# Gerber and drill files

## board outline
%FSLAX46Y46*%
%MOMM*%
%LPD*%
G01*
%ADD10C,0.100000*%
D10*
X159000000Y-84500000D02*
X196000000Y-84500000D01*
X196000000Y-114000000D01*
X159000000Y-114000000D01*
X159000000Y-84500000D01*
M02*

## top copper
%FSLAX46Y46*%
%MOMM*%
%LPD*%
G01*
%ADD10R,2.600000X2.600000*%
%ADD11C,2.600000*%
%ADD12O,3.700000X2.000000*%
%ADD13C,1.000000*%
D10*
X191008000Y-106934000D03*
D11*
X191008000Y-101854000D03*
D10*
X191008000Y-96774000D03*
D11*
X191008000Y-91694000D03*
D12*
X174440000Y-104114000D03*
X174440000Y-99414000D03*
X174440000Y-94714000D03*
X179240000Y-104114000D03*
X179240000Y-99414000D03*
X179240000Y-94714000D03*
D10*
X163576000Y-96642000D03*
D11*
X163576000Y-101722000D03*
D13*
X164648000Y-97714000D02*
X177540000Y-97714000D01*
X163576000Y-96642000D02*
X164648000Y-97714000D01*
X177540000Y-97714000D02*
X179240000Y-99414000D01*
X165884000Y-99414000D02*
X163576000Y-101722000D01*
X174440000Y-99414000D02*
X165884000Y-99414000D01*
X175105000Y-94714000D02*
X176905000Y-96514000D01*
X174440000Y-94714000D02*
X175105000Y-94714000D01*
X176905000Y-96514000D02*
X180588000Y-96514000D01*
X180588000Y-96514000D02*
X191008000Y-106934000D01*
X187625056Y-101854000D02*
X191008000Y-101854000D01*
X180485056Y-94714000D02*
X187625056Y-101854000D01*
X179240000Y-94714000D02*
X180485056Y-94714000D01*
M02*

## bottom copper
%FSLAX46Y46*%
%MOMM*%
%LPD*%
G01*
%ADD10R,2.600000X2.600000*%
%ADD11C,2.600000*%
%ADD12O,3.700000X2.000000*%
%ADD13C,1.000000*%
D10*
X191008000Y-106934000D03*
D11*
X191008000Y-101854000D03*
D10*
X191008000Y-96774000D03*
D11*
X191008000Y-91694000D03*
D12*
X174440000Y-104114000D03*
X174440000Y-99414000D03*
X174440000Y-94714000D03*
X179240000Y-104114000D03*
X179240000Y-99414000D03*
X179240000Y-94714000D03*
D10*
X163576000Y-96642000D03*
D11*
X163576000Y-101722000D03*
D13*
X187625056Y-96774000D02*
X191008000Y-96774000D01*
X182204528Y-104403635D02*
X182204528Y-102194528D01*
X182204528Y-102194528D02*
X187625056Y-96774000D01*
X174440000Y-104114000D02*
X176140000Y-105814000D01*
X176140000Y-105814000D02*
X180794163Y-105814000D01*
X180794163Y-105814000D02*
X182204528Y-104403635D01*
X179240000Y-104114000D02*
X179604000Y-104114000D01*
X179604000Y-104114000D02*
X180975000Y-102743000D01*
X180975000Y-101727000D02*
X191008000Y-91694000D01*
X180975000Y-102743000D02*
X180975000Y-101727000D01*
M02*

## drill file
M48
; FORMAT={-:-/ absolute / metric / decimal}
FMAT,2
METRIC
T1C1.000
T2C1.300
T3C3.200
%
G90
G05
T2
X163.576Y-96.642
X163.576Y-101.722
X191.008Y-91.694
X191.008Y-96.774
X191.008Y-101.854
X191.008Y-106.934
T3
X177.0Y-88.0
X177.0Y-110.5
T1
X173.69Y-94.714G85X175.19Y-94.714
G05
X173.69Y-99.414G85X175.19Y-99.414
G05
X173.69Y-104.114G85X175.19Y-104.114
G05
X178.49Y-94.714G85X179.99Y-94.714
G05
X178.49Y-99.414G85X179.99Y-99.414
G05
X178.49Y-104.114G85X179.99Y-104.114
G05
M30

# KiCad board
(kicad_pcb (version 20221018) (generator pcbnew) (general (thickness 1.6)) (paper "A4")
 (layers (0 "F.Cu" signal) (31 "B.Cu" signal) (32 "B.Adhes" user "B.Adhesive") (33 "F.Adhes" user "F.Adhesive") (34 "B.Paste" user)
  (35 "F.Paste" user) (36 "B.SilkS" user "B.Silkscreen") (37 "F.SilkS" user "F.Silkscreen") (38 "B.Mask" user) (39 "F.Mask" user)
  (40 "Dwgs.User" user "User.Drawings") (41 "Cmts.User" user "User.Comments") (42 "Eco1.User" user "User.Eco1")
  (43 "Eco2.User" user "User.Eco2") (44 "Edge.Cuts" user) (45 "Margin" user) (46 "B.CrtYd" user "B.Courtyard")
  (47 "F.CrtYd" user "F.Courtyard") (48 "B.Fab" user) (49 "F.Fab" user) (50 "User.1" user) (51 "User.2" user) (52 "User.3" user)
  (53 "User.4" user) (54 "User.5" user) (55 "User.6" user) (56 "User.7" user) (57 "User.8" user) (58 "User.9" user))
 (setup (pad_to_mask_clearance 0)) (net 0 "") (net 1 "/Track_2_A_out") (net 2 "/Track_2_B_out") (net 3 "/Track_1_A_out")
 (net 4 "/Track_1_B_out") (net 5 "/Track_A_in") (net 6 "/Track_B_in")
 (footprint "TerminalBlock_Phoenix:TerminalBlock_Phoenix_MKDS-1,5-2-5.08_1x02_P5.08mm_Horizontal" (layer "F.Cu") (at 191.008 106.934 90)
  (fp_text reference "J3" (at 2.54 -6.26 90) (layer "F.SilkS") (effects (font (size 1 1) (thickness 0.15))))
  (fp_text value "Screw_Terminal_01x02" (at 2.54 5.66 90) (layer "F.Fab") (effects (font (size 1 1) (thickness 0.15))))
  (pad "1" thru_hole rect (at 0 0 90) (size 2.6 2.6) (drill 1.3) (layers "*.Cu" "*.Mask") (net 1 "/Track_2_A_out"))
  (pad "2" thru_hole circle (at 5.08 0 90) (size 2.6 2.6) (drill 1.3) (layers "*.Cu" "*.Mask") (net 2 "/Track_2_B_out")))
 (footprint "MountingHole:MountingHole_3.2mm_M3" (layer "F.Cu") (at 177 88)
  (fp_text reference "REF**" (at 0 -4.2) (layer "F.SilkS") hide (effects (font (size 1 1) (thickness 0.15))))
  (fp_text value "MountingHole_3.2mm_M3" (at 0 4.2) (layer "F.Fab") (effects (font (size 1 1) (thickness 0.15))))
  (pad "" np_thru_hole circle (at 0 0) (size 3.2 3.2) (drill 3.2) (layers "F&B.Cu" "*.Mask")))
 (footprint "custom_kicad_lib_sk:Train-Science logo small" (layer "F.Cu") (at 165.481 109.093 -90)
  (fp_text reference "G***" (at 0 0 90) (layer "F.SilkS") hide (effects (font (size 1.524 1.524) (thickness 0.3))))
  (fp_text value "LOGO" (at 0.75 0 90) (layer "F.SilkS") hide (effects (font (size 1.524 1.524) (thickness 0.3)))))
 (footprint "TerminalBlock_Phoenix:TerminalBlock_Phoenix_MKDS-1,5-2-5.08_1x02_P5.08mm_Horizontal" (layer "F.Cu") (at 191.008 96.774 90)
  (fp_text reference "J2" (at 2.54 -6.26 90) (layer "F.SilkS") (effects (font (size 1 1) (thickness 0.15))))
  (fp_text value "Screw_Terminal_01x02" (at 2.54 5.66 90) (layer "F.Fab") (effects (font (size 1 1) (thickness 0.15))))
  (pad "1" thru_hole rect (at 0 0 90) (size 2.6 2.6) (drill 1.3) (layers "*.Cu" "*.Mask") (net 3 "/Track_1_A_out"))
  (pad "2" thru_hole circle (at 5.08 0 90) (size 2.6 2.6) (drill 1.3) (layers "*.Cu" "*.Mask") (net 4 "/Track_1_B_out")))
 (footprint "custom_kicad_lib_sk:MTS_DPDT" (layer "F.Cu") (at 177.44 95.414 90)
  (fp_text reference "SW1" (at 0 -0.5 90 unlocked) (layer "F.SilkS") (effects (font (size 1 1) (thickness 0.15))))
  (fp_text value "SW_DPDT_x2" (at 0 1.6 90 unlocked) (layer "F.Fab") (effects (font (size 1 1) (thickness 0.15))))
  (pad "1" thru_hole oval (at -8.7 -3 90) (size 2 3.7) (drill oval 1 2.5) (layers "*.Cu" "*.Mask") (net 3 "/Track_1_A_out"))
  (pad "2" thru_hole oval (at -4 -3 90) (size 2 3.7) (drill oval 1 2.5) (layers "*.Cu" "*.Mask") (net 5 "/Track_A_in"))
  (pad "3" thru_hole oval (at 0.7 -3 90) (size 2 3.7) (drill oval 1 2.5) (layers "*.Cu" "*.Mask") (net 1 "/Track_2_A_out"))
  (pad "4" thru_hole oval (at -8.7 1.8 90) (size 2 3.7) (drill oval 1 2.5) (layers "*.Cu" "*.Mask") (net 4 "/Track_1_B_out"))
  (pad "5" thru_hole oval (at -4 1.8 90) (size 2 3.7) (drill oval 1 2.5) (layers "*.Cu" "*.Mask") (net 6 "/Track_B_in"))
  (pad "6" thru_hole oval (at 0.7 1.8 90) (size 2 3.7) (drill oval 1 2.5) (layers "*.Cu" "*.Mask") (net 2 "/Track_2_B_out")))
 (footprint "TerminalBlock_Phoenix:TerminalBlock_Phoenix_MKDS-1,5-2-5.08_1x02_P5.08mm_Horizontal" (layer "F.Cu") (at 163.576 96.642 -90)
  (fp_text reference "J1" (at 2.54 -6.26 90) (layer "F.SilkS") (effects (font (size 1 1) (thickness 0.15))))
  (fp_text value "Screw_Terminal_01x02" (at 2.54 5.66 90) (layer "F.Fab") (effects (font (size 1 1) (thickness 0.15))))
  (pad "1" thru_hole rect (at 0 0 270) (size 2.6 2.6) (drill 1.3) (layers "*.Cu" "*.Mask") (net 6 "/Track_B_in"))
  (pad "2" thru_hole circle (at 5.08 0 270) (size 2.6 2.6) (drill 1.3) (layers "*.Cu" "*.Mask") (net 5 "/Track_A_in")))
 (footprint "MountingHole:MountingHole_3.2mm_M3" (layer "F.Cu") (at 177 110.5)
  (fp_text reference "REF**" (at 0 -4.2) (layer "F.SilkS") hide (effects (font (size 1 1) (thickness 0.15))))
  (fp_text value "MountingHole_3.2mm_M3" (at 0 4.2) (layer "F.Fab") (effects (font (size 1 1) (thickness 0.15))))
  (pad "" np_thru_hole circle (at 0 0) (size 3.2 3.2) (drill 3.2) (layers "*.Cu" "*.Mask")))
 (gr_rect (start 159 84.5) (end 196 114) (stroke (width 0.1) (type default)) (fill none) (layer "Edge.Cuts"))
 (segment (start 164.648 97.714) (end 177.54 97.714) (width 1) (layer "F.Cu") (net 6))
 (segment (start 163.576 96.642) (end 164.648 97.714) (width 1) (layer "F.Cu") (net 6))
 (segment (start 177.54 97.714) (end 179.24 99.414) (width 1) (layer "F.Cu") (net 6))
 (segment (start 165.884 99.414) (end 163.576 101.722) (width 1) (layer "F.Cu") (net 5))
 (segment (start 174.44 99.414) (end 165.884 99.414) (width 1) (layer "F.Cu") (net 5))
 (segment (start 187.625056 96.774) (end 191.008 96.774) (width 1) (layer "B.Cu") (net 3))
 (segment (start 182.204528 104.403635) (end 182.204528 102.194528) (width 1) (layer "B.Cu") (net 3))
 (segment (start 182.204528 102.194528) (end 187.625056 96.774) (width 1) (layer "B.Cu") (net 3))
 (segment (start 174.44 104.114) (end 176.14 105.814) (width 1) (layer "B.Cu") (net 3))
 (segment (start 176.14 105.814) (end 180.794163 105.814) (width 1) (layer "B.Cu") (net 3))
 (segment (start 180.794163 105.814) (end 182.204528 104.403635) (width 1) (layer "B.Cu") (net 3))
 (segment (start 179.24 104.114) (end 179.604 104.114) (width 1) (layer "B.Cu") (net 4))
 (segment (start 179.604 104.114) (end 180.975 102.743) (width 1) (layer "B.Cu") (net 4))
 (segment (start 180.975 101.727) (end 191.008 91.694) (width 1) (layer "B.Cu") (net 4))
 (segment (start 180.975 102.743) (end 180.975 101.727) (width 1) (layer "B.Cu") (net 4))
 (segment (start 175.105 94.714) (end 176.905 96.514) (width 1) (layer "F.Cu") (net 1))
 (segment (start 174.44 94.714) (end 175.105 94.714) (width 1) (layer "F.Cu") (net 1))
 (segment (start 176.905 96.514) (end 180.588 96.514) (width 1) (layer "F.Cu") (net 1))
 (segment (start 180.588 96.514) (end 191.008 106.934) (width 1) (layer "F.Cu") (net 1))
 (segment (start 187.625056 101.854) (end 191.008 101.854) (width 1) (layer "F.Cu") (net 2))
 (segment (start 180.485056 94.714) (end 187.625056 101.854) (width 1) (layer "F.Cu") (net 2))
 (segment (start 179.24 94.714) (end 180.485056 94.714) (width 1) (layer "F.Cu") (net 2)))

